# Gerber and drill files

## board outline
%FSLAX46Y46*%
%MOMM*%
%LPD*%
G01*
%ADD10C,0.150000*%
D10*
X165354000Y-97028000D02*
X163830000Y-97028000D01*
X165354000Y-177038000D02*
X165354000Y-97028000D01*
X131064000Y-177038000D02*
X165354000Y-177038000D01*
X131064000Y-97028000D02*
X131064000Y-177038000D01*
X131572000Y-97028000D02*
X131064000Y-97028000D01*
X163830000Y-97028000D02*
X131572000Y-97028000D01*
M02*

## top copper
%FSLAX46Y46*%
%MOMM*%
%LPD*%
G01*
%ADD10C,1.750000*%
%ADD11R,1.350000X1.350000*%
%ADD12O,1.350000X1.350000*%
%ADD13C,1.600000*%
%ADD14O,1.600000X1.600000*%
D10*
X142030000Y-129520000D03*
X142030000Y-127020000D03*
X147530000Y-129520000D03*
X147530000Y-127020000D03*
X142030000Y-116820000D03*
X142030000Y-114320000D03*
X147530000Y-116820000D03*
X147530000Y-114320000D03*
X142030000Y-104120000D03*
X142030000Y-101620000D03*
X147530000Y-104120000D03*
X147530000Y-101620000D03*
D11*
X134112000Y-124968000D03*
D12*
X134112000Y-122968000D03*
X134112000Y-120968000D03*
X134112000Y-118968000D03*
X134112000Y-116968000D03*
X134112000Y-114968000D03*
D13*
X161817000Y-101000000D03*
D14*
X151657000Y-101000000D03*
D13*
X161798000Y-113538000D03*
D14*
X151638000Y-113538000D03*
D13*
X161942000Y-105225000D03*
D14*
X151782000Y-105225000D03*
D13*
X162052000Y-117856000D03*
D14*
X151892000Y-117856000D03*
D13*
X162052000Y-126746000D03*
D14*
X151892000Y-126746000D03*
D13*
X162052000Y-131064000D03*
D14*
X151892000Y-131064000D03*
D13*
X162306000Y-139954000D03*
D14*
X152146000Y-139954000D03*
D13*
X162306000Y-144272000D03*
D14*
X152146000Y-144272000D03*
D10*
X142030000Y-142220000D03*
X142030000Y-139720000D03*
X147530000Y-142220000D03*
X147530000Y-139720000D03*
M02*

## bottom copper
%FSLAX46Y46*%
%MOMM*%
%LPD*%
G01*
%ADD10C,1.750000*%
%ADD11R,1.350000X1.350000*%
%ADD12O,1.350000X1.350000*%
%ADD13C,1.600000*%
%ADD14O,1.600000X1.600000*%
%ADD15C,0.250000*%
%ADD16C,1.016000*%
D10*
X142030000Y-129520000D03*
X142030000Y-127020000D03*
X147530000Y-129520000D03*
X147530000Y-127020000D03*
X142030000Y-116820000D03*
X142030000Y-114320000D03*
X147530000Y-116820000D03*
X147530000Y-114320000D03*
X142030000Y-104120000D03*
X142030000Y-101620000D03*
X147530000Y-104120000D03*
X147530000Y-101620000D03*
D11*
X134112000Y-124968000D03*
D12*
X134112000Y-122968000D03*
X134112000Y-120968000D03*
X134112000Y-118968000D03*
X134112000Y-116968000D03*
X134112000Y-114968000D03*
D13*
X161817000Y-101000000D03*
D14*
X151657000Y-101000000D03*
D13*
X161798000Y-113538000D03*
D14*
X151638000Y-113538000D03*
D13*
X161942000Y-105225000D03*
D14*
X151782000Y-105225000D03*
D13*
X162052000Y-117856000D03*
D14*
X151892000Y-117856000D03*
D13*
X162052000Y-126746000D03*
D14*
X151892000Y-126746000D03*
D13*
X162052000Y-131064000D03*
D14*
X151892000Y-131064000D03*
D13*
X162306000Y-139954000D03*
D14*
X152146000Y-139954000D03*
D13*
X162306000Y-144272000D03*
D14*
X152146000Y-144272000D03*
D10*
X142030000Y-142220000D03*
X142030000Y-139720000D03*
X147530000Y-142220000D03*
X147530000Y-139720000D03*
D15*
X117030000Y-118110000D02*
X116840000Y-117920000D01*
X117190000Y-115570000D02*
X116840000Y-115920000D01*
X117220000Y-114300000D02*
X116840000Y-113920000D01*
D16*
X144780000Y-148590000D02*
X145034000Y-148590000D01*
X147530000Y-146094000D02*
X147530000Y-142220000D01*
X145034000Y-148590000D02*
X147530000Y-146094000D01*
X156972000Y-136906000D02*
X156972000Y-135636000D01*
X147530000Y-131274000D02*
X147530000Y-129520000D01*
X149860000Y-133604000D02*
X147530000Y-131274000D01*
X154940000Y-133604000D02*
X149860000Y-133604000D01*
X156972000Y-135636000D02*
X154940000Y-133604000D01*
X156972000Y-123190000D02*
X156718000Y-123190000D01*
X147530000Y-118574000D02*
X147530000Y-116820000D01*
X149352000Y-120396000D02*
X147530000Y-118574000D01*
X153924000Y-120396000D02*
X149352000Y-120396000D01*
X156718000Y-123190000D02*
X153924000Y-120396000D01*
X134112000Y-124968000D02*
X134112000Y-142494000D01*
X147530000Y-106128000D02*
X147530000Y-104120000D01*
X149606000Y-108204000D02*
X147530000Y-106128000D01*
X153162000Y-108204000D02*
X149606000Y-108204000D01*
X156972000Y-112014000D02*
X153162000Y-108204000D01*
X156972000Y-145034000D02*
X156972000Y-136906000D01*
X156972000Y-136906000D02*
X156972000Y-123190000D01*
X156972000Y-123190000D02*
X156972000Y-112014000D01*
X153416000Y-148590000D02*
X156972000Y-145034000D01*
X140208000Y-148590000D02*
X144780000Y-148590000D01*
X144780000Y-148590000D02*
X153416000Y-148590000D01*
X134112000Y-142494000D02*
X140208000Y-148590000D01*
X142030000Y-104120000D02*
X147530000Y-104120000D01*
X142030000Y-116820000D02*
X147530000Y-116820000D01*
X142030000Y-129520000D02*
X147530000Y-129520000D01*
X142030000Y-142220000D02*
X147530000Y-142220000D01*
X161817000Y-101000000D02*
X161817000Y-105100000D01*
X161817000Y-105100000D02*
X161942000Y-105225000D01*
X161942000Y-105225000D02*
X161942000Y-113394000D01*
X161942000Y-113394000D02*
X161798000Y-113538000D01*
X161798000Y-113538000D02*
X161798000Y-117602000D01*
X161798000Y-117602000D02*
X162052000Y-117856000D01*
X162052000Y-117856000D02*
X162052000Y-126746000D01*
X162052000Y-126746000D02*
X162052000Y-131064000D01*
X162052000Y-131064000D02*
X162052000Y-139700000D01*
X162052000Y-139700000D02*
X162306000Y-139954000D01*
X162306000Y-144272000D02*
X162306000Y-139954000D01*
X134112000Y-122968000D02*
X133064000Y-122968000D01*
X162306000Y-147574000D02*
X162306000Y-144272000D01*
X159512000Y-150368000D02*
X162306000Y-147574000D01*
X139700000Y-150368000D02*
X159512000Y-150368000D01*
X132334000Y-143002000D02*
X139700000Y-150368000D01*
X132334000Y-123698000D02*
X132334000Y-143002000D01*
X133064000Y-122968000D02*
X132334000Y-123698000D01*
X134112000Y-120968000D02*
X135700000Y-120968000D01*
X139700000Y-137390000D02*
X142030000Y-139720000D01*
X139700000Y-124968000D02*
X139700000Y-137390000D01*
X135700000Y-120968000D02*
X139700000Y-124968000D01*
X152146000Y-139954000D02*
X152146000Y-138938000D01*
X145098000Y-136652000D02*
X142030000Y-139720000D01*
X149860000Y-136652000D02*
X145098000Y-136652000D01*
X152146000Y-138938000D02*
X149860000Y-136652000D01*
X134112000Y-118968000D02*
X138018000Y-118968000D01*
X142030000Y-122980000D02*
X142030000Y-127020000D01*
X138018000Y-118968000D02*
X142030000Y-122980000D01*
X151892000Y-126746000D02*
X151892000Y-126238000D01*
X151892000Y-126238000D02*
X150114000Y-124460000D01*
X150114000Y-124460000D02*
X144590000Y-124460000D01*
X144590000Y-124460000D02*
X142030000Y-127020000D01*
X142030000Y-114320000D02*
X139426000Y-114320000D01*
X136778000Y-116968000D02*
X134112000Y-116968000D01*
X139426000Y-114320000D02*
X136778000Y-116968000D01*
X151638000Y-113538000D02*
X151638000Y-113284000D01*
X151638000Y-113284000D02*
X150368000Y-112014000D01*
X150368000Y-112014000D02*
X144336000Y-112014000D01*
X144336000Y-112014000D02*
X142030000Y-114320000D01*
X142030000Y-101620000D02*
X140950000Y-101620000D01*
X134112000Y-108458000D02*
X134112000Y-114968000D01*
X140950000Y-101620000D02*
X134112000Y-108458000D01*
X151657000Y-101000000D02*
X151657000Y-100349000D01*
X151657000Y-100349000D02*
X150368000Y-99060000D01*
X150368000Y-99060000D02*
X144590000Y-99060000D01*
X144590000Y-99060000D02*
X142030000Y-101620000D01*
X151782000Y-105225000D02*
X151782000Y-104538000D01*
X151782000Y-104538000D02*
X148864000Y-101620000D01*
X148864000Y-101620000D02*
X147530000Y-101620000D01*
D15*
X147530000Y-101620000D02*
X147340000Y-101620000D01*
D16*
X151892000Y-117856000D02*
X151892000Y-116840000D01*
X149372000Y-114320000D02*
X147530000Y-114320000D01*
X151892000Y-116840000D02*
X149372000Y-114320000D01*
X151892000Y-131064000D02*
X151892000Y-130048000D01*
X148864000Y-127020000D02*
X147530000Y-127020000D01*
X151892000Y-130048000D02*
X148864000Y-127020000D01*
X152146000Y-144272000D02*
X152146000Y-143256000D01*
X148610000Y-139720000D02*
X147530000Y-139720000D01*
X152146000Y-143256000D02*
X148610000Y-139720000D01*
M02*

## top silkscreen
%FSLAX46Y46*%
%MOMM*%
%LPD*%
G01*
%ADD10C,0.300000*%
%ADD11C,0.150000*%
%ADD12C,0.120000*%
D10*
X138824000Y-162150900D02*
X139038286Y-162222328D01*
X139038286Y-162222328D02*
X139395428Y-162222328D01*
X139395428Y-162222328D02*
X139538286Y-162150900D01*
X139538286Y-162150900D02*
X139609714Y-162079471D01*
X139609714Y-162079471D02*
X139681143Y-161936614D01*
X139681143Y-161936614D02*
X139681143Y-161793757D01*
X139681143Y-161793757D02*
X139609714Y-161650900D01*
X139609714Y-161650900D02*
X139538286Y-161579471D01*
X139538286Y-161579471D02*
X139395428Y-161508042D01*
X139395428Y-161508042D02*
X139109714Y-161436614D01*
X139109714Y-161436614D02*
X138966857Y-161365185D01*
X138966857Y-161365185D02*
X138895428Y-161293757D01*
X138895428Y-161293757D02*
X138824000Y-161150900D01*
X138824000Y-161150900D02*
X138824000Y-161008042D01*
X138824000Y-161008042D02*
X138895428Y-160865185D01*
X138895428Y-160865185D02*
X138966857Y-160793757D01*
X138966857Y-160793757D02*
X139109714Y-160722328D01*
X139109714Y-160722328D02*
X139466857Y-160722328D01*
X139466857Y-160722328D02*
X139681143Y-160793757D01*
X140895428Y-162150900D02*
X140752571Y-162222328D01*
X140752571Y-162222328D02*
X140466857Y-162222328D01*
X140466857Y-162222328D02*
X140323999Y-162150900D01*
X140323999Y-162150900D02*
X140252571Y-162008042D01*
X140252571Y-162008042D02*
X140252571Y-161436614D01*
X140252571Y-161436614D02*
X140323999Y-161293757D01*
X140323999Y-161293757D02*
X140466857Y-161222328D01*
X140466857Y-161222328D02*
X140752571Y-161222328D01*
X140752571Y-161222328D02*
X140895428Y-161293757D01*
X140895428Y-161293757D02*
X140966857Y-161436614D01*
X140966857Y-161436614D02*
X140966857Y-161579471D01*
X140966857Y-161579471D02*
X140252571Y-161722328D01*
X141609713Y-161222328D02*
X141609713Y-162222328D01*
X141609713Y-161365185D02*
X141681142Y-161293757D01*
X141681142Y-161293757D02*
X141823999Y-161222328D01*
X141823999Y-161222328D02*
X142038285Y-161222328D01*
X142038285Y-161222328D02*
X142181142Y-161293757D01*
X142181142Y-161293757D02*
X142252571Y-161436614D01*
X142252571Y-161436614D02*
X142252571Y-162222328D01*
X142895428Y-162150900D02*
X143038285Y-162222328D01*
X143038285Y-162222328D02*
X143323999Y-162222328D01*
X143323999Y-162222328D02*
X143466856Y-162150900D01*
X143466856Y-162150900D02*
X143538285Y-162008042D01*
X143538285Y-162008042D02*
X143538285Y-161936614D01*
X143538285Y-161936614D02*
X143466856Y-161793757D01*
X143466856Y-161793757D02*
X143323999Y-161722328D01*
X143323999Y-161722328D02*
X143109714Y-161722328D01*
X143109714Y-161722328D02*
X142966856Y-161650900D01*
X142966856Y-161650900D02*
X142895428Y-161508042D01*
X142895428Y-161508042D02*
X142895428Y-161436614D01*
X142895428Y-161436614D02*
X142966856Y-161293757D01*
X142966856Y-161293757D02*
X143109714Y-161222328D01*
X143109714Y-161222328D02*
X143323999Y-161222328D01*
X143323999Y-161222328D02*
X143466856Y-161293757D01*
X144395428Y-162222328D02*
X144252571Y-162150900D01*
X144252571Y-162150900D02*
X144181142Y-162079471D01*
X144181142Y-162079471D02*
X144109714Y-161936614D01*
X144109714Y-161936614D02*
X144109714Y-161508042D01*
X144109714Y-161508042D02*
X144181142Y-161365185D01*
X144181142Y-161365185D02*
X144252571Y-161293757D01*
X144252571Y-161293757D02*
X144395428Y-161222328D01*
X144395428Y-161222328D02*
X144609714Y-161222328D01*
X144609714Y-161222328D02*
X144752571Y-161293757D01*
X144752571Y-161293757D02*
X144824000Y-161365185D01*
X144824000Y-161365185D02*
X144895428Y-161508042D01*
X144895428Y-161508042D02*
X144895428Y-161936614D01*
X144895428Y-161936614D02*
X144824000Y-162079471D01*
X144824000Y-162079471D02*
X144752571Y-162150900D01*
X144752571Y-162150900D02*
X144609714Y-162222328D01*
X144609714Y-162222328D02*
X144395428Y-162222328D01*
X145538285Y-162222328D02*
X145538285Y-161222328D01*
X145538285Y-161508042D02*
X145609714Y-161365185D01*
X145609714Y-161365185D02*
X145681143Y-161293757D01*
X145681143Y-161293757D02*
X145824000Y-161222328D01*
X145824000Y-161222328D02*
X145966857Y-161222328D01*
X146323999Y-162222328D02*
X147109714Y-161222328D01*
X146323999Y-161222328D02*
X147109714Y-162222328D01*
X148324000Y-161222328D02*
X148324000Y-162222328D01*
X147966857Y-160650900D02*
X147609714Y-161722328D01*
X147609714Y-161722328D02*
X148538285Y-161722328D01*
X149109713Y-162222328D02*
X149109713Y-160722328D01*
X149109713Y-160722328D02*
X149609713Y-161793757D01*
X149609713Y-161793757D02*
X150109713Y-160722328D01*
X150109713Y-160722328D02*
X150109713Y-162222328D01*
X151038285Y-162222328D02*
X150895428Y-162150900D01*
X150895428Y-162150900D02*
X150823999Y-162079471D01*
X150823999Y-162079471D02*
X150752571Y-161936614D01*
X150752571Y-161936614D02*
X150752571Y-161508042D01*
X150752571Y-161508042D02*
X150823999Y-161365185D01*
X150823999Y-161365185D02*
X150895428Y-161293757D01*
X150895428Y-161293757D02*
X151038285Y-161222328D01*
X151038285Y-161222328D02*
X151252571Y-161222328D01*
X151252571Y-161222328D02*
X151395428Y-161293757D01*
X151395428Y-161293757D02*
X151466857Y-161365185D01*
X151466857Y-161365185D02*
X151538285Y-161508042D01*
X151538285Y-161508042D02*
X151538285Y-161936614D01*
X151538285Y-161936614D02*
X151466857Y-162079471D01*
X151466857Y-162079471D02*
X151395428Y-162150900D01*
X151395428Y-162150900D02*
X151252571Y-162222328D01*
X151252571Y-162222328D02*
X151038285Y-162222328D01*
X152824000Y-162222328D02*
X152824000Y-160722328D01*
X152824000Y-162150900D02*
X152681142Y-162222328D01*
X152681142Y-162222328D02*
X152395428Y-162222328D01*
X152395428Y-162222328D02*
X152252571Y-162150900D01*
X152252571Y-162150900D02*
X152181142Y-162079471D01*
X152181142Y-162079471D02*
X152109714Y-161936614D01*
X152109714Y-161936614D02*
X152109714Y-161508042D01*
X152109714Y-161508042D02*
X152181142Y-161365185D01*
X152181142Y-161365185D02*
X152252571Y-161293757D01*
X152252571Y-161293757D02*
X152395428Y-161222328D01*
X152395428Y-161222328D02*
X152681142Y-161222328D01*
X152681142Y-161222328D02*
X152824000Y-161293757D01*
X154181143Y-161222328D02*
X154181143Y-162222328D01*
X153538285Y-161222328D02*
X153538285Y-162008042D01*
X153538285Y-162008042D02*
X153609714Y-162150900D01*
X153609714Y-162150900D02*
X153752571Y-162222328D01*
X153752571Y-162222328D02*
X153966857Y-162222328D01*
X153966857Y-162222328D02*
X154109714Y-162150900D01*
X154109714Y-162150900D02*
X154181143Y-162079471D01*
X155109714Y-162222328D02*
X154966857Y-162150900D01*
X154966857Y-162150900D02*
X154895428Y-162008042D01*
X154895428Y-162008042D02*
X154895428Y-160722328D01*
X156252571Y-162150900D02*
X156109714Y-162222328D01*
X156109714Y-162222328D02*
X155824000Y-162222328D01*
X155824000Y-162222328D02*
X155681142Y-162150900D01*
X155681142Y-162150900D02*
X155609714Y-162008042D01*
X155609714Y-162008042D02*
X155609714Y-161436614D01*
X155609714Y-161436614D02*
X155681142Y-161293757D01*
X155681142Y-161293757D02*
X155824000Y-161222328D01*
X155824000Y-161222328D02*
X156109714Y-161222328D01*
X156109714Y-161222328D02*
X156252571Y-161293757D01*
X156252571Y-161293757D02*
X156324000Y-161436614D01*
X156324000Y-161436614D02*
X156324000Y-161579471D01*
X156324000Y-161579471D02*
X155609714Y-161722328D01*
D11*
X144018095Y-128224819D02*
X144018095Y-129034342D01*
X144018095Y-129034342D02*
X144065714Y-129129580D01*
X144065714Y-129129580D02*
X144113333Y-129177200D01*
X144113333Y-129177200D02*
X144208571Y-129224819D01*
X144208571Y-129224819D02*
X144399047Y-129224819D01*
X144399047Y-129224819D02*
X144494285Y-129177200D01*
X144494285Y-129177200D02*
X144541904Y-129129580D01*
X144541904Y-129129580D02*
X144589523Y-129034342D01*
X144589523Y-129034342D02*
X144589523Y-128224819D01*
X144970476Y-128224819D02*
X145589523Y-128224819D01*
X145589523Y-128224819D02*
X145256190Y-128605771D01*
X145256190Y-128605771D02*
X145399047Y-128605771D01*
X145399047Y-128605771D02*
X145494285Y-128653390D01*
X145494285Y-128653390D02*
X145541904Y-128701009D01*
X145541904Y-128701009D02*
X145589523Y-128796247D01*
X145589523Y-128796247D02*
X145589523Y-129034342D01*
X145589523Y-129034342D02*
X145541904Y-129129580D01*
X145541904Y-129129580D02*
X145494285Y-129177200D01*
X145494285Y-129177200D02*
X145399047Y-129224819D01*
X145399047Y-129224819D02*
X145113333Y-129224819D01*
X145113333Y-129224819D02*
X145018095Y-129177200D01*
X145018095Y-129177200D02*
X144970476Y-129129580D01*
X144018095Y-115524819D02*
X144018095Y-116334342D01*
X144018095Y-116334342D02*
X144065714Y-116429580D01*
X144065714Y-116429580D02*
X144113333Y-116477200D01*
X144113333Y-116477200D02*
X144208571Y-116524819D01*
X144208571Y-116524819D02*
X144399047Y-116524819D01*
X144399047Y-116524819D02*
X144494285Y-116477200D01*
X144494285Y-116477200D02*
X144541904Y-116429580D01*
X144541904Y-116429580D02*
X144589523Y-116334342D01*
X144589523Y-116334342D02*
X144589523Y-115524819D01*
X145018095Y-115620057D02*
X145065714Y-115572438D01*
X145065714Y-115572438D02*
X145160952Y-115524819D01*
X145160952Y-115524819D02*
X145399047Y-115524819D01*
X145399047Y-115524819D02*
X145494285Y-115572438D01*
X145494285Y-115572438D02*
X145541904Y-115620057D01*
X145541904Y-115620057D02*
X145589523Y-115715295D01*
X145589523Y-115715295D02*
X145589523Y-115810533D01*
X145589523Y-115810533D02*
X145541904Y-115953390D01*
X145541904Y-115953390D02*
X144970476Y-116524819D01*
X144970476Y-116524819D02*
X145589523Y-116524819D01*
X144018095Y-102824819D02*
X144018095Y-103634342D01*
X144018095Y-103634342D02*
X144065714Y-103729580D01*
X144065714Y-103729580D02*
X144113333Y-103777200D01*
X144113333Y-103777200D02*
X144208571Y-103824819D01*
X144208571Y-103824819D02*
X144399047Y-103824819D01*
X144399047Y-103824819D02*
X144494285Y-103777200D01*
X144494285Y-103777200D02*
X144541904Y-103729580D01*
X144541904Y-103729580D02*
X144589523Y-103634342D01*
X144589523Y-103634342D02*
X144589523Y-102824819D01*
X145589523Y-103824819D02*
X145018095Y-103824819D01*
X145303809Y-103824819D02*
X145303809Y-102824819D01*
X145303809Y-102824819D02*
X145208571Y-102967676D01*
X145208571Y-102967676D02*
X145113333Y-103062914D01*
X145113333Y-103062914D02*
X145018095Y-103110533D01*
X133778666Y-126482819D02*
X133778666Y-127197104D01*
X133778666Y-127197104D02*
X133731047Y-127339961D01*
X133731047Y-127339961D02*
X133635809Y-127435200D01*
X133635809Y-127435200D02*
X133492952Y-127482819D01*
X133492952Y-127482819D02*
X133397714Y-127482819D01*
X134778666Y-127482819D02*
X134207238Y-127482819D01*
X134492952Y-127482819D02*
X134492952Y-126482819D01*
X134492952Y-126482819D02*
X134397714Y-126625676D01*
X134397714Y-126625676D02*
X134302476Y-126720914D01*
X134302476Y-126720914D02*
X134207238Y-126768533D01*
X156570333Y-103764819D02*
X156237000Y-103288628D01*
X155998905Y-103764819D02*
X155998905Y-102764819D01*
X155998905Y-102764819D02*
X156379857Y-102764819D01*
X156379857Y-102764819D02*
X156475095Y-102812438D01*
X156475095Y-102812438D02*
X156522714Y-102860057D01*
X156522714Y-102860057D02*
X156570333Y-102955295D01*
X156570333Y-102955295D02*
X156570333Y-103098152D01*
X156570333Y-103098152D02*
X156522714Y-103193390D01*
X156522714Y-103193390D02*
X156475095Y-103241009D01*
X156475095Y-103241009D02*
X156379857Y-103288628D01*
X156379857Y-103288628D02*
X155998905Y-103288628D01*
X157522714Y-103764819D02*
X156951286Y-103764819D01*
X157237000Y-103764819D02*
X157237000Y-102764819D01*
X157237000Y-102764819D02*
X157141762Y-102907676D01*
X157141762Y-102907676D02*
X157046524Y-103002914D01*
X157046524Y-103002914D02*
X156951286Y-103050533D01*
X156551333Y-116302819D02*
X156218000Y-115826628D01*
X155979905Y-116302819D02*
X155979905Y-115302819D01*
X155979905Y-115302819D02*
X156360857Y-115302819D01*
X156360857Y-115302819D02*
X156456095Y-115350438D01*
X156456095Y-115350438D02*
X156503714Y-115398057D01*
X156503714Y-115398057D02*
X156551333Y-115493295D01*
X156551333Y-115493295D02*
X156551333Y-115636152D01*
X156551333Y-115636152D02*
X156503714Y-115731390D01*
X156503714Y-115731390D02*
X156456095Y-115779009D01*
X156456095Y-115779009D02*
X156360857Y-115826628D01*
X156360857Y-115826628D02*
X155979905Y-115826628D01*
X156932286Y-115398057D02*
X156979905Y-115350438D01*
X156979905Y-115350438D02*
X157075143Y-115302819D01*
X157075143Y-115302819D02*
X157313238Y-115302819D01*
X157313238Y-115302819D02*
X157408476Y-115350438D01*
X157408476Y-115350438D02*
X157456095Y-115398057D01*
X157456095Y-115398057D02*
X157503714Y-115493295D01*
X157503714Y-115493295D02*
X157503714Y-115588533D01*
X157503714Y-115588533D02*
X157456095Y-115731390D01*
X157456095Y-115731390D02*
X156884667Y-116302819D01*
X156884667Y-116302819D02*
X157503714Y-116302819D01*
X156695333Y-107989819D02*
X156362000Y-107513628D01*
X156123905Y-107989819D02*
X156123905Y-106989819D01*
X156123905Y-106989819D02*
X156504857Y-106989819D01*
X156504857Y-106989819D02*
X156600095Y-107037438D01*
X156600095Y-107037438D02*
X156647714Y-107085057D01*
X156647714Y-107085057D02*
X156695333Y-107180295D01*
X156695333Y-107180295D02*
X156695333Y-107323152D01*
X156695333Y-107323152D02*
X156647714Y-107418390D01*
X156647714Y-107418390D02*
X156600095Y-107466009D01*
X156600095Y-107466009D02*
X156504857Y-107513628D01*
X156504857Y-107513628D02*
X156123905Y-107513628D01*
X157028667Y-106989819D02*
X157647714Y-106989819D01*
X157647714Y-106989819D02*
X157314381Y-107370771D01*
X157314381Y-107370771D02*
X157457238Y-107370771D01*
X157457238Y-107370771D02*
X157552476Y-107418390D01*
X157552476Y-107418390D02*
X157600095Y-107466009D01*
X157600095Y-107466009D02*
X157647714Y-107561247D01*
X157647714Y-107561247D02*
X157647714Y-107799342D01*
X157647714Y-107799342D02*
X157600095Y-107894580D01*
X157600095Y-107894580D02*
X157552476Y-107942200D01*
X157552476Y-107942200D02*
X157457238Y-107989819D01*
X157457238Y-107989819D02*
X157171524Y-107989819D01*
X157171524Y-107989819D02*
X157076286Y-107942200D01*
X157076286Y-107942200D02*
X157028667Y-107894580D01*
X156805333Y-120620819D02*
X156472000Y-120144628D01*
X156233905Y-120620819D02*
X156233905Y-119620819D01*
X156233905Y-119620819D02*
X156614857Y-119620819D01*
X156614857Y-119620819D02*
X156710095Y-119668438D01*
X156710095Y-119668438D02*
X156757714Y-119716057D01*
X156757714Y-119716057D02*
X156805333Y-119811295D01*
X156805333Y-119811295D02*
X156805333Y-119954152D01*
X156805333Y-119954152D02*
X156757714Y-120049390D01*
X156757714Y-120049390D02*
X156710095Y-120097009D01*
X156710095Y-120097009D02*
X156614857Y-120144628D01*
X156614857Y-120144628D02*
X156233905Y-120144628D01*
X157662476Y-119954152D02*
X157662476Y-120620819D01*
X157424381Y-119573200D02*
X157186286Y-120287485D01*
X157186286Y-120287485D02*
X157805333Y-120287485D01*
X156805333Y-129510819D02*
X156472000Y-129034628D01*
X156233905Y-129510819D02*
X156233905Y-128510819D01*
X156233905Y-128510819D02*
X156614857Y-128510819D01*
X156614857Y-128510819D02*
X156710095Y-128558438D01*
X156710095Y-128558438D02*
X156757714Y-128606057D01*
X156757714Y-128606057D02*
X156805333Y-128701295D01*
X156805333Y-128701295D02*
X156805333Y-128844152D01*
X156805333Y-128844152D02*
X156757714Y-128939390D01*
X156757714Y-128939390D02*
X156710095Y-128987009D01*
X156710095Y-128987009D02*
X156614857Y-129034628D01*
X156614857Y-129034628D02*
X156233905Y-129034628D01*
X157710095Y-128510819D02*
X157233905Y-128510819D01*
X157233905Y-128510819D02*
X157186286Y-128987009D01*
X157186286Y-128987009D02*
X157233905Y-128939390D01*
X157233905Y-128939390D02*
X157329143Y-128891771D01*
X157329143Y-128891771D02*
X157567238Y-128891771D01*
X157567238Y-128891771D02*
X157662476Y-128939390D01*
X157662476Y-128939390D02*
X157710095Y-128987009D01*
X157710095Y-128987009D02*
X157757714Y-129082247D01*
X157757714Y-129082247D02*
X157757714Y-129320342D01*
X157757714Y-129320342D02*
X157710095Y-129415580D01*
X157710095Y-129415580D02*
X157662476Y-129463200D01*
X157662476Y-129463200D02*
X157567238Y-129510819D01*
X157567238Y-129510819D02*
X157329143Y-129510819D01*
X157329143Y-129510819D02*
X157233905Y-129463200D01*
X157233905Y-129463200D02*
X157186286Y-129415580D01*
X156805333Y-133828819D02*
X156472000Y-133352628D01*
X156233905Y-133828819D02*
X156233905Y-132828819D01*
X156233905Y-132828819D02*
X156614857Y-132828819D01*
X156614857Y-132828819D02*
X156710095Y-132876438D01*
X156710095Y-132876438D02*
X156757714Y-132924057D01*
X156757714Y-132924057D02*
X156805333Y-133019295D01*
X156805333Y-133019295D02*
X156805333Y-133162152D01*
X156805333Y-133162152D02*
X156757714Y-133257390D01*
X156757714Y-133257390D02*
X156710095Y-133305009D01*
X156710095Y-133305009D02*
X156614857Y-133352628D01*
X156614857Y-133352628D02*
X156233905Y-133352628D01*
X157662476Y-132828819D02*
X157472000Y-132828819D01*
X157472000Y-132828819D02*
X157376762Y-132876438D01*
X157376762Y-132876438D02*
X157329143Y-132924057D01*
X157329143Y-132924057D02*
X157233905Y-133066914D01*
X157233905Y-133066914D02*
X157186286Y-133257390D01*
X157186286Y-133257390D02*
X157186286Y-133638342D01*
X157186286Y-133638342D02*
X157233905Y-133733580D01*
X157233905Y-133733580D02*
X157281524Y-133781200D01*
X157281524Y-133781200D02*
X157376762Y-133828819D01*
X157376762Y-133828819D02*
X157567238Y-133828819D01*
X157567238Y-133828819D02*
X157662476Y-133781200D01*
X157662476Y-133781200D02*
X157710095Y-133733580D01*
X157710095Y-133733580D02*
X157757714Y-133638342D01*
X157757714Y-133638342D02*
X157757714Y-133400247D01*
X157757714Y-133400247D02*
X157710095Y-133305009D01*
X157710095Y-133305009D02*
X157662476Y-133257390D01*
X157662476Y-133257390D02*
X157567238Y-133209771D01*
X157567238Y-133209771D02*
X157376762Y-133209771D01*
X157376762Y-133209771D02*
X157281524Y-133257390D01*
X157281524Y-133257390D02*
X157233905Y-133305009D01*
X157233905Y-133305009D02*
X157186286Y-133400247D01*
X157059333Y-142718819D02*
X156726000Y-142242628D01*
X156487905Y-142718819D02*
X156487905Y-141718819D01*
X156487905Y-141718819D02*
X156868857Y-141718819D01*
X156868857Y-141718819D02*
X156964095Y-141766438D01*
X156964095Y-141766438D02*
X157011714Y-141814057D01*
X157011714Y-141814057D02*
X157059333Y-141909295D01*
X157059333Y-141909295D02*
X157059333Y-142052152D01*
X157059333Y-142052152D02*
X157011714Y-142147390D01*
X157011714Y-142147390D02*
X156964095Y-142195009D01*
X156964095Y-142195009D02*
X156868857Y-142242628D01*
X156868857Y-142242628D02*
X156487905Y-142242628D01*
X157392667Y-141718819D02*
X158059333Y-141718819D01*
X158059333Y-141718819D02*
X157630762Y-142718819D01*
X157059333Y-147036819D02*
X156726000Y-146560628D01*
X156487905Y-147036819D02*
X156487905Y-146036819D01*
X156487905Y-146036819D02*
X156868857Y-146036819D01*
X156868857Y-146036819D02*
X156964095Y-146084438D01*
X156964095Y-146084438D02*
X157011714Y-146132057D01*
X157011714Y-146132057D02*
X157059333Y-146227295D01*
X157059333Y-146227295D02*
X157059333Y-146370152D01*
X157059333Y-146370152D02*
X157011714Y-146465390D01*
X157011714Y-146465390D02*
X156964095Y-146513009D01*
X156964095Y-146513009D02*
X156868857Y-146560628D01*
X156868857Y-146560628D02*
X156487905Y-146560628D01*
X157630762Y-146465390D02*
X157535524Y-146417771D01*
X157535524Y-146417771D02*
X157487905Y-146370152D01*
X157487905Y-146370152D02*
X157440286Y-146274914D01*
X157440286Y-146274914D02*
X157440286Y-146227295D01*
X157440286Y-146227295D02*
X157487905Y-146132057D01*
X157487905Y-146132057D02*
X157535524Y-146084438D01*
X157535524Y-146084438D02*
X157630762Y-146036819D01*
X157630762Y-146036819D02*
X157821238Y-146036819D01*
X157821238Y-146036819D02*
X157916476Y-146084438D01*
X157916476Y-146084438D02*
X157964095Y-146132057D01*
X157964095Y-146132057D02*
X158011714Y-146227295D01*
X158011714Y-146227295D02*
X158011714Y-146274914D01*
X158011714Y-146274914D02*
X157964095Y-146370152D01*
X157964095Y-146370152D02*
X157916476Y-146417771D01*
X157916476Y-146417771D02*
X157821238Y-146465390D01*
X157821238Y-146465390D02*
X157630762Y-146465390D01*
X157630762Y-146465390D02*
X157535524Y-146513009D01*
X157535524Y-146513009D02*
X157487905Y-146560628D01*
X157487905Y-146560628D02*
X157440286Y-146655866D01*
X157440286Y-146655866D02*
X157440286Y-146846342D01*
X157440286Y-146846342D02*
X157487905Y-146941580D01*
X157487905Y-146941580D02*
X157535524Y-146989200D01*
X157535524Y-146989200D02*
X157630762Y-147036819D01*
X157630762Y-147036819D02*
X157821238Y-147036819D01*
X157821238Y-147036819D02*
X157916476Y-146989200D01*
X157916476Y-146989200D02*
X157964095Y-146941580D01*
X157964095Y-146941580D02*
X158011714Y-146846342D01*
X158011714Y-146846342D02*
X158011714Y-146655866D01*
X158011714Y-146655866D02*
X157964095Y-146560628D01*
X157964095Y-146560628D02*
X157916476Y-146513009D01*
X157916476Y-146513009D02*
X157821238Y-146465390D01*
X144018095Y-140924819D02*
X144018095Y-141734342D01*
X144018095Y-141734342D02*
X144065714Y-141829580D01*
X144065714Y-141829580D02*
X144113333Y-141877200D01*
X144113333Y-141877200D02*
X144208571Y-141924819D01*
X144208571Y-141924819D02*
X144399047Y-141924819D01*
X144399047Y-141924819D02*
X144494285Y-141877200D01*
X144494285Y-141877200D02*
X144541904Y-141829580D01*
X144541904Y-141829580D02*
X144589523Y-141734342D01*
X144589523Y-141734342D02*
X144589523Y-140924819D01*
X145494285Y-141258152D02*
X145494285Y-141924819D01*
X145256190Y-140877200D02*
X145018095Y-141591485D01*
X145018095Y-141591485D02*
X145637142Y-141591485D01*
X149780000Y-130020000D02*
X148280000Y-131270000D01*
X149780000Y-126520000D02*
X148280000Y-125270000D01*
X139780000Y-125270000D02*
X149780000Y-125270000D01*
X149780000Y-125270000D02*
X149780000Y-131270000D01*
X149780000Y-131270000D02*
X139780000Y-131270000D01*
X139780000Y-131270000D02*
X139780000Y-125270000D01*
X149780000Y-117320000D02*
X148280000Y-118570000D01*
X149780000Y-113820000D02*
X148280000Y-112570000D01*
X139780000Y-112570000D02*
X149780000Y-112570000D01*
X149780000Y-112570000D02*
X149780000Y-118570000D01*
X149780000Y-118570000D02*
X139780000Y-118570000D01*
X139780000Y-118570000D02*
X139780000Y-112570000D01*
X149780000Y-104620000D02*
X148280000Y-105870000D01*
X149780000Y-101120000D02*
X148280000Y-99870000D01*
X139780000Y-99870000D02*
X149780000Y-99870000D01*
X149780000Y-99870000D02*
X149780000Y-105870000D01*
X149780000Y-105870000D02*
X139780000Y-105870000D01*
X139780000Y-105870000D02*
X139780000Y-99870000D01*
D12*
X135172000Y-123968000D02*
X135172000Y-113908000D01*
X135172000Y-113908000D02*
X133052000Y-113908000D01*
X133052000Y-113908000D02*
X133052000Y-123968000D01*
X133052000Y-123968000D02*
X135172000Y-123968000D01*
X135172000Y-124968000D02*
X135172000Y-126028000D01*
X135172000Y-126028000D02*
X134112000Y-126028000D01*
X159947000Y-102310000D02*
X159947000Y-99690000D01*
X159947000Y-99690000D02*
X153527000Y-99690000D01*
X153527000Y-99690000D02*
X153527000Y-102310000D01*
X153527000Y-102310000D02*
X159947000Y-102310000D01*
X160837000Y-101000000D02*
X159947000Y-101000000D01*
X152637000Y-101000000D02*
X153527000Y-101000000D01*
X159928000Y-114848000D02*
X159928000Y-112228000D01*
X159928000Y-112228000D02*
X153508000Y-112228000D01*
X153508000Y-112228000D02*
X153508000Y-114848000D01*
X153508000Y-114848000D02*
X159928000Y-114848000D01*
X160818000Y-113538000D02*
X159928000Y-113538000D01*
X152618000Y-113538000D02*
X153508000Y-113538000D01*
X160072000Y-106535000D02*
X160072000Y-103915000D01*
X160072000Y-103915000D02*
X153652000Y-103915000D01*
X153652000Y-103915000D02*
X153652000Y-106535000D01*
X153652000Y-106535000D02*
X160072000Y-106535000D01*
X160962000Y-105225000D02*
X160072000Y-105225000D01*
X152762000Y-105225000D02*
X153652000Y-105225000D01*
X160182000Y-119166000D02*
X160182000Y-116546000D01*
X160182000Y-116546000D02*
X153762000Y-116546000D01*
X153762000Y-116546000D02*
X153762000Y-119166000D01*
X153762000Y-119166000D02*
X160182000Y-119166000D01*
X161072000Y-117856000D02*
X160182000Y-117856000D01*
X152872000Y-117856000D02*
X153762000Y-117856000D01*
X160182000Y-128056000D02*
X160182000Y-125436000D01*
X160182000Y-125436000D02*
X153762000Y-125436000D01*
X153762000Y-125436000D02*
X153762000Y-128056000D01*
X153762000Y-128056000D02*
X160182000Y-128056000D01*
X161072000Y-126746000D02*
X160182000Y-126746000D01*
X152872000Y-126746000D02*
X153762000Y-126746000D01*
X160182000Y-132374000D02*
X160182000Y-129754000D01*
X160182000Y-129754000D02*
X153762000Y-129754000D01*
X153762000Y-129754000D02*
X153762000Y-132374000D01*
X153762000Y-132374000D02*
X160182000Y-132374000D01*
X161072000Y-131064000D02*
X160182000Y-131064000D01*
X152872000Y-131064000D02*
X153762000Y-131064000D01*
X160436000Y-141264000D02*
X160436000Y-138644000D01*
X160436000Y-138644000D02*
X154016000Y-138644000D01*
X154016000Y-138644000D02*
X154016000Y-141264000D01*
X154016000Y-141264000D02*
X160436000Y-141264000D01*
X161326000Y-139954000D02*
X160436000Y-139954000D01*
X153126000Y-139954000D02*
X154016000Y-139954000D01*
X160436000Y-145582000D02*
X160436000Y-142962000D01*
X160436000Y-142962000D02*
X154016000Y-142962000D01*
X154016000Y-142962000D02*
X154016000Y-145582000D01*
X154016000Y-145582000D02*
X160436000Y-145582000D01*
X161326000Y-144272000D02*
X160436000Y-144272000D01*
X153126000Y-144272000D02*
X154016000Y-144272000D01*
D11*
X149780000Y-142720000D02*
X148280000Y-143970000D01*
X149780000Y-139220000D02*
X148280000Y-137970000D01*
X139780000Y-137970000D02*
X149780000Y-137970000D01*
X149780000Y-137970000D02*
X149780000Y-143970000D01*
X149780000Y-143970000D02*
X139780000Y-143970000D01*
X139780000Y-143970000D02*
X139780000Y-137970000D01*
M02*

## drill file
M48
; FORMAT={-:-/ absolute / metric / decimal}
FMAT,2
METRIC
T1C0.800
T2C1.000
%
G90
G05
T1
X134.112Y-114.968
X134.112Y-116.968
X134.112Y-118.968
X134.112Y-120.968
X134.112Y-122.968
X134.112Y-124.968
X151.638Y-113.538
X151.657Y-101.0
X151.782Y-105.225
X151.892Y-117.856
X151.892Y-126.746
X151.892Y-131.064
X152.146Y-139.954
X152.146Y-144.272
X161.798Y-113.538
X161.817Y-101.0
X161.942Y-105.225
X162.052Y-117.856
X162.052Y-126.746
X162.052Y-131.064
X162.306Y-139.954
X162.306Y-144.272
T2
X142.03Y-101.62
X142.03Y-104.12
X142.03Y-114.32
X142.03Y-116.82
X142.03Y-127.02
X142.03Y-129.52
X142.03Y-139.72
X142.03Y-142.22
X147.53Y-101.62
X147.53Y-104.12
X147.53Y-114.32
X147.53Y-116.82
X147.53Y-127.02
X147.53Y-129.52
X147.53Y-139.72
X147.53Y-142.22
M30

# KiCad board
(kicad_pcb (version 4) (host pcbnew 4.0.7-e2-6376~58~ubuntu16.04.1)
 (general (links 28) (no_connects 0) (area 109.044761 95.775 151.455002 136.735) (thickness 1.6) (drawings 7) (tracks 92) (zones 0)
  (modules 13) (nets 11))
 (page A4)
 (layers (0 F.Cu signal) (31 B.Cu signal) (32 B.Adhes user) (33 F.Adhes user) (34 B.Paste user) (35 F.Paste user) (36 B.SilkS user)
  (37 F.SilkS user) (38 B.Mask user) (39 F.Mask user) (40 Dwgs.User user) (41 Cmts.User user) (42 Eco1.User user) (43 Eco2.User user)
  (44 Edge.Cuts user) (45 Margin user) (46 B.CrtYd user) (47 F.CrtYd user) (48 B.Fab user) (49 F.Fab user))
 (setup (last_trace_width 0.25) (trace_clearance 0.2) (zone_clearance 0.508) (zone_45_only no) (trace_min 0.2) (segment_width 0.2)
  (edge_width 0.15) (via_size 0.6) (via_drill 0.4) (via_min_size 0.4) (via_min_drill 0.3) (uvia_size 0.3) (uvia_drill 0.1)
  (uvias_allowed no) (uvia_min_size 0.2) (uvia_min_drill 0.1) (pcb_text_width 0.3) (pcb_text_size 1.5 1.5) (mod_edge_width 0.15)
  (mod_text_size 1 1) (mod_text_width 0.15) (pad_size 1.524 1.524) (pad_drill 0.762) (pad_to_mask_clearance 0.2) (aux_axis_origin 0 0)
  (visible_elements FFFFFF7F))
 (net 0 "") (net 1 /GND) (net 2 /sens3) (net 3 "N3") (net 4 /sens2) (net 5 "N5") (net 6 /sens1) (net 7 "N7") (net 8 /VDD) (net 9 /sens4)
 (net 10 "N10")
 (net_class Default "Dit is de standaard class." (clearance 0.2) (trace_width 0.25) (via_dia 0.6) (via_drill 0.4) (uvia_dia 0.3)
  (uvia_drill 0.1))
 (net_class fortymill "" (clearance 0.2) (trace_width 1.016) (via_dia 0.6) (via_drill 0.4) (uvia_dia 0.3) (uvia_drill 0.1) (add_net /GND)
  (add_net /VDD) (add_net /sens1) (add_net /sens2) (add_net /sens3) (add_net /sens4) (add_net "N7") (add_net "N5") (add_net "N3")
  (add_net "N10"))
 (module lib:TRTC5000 (layer F.Cu) (at 144.78 128.27)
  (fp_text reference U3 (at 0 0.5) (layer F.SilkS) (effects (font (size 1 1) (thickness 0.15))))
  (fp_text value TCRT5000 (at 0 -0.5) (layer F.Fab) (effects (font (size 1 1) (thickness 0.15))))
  (fp_line (start 5 1.75) (end 3.5 3) (layer F.SilkS) (width 0.15))
  (fp_line (start 5 -1.75) (end 3.5 -3) (layer F.SilkS) (width 0.15))
  (fp_line (start -5 -3) (end 5 -3) (layer F.SilkS) (width 0.15))
  (fp_line (start 5 -3) (end 5 3) (layer F.SilkS) (width 0.15))
  (fp_line (start 5 3) (end -5 3) (layer F.SilkS) (width 0.15))
  (fp_line (start -5 3) (end -5 -3) (layer F.SilkS) (width 0.15))
  (pad 2 thru_hole circle (at -2.75 1.25) (size 1.75 1.75) (drill 1) (layers *.Cu *.Mask) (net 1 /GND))
  (pad 1 thru_hole circle (at -2.75 -1.25) (size 1.75 1.75) (drill 1) (layers *.Cu *.Mask) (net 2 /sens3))
  (pad 4 thru_hole circle (at 2.75 1.25) (size 1.75 1.75) (drill 1) (layers *.Cu *.Mask) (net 1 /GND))
  (pad 3 thru_hole circle (at 2.75 -1.25) (size 1.75 1.75) (drill 1) (layers *.Cu *.Mask) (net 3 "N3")))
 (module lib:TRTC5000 (layer F.Cu) (at 144.78 115.57)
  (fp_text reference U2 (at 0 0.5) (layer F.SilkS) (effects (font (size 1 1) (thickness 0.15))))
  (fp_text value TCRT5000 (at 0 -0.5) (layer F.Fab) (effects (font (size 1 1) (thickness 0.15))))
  (fp_line (start 5 1.75) (end 3.5 3) (layer F.SilkS) (width 0.15))
  (fp_line (start 5 -1.75) (end 3.5 -3) (layer F.SilkS) (width 0.15))
  (fp_line (start -5 -3) (end 5 -3) (layer F.SilkS) (width 0.15))
  (fp_line (start 5 -3) (end 5 3) (layer F.SilkS) (width 0.15))
  (fp_line (start 5 3) (end -5 3) (layer F.SilkS) (width 0.15))
  (fp_line (start -5 3) (end -5 -3) (layer F.SilkS) (width 0.15))
  (pad 2 thru_hole circle (at -2.75 1.25) (size 1.75 1.75) (drill 1) (layers *.Cu *.Mask) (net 1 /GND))
  (pad 1 thru_hole circle (at -2.75 -1.25) (size 1.75 1.75) (drill 1) (layers *.Cu *.Mask) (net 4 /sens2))
  (pad 4 thru_hole circle (at 2.75 1.25) (size 1.75 1.75) (drill 1) (layers *.Cu *.Mask) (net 1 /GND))
  (pad 3 thru_hole circle (at 2.75 -1.25) (size 1.75 1.75) (drill 1) (layers *.Cu *.Mask) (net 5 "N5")))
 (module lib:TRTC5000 (layer F.Cu) (at 144.78 102.87)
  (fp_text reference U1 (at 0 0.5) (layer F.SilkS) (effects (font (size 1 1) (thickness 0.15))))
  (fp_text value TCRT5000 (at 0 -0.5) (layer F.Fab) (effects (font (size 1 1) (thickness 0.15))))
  (fp_line (start 5 1.75) (end 3.5 3) (layer F.SilkS) (width 0.15))
  (fp_line (start 5 -1.75) (end 3.5 -3) (layer F.SilkS) (width 0.15))
  (fp_line (start -5 -3) (end 5 -3) (layer F.SilkS) (width 0.15))
  (fp_line (start 5 -3) (end 5 3) (layer F.SilkS) (width 0.15))
  (fp_line (start 5 3) (end -5 3) (layer F.SilkS) (width 0.15))
  (fp_line (start -5 3) (end -5 -3) (layer F.SilkS) (width 0.15))
  (pad 2 thru_hole circle (at -2.75 1.25) (size 1.75 1.75) (drill 1) (layers *.Cu *.Mask) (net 1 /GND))
  (pad 1 thru_hole circle (at -2.75 -1.25) (size 1.75 1.75) (drill 1) (layers *.Cu *.Mask) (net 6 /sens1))
  (pad 4 thru_hole circle (at 2.75 1.25) (size 1.75 1.75) (drill 1) (layers *.Cu *.Mask) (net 1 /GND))
  (pad 3 thru_hole circle (at 2.75 -1.25) (size 1.75 1.75) (drill 1) (layers *.Cu *.Mask) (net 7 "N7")))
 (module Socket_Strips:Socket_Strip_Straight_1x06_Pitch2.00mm (layer F.Cu) (at 134.112 124.968 180)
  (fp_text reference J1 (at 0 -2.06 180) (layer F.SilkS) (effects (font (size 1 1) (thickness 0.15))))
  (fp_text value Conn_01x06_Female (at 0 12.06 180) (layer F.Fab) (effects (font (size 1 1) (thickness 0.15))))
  (fp_line (start -1.06 1) (end -1.06 11.06) (layer F.SilkS) (width 0.12))
  (fp_line (start -1.06 11.06) (end 1.06 11.06) (layer F.SilkS) (width 0.12))
  (fp_line (start 1.06 11.06) (end 1.06 1) (layer F.SilkS) (width 0.12))
  (fp_line (start 1.06 1) (end -1.06 1) (layer F.SilkS) (width 0.12))
  (fp_line (start -1.06 0) (end -1.06 -1.06) (layer F.SilkS) (width 0.12))
  (fp_line (start -1.06 -1.06) (end 0 -1.06) (layer F.SilkS) (width 0.12))
  (pad 1 thru_hole rect (at 0 0 180) (size 1.35 1.35) (drill 0.8) (layers *.Cu *.Mask) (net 1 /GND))
  (pad 2 thru_hole oval (at 0 2 180) (size 1.35 1.35) (drill 0.8) (layers *.Cu *.Mask) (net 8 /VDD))
  (pad 3 thru_hole oval (at 0 4 180) (size 1.35 1.35) (drill 0.8) (layers *.Cu *.Mask) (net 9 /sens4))
  (pad 4 thru_hole oval (at 0 6 180) (size 1.35 1.35) (drill 0.8) (layers *.Cu *.Mask) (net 2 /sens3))
  (pad 5 thru_hole oval (at 0 8 180) (size 1.35 1.35) (drill 0.8) (layers *.Cu *.Mask) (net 4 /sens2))
  (pad 6 thru_hole oval (at 0 10 180) (size 1.35 1.35) (drill 0.8) (layers *.Cu *.Mask) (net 6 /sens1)))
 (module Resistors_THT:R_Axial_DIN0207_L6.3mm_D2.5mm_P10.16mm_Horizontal (layer F.Cu) (at 161.817 101 180)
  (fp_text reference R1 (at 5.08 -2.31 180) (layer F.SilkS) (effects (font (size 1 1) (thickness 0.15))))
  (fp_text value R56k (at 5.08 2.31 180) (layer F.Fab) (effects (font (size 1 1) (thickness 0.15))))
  (fp_line (start 1.87 -1.31) (end 1.87 1.31) (layer F.SilkS) (width 0.12))
  (fp_line (start 1.87 1.31) (end 8.29 1.31) (layer F.SilkS) (width 0.12))
  (fp_line (start 8.29 1.31) (end 8.29 -1.31) (layer F.SilkS) (width 0.12))
  (fp_line (start 8.29 -1.31) (end 1.87 -1.31) (layer F.SilkS) (width 0.12))
  (fp_line (start 0.98 0) (end 1.87 0) (layer F.SilkS) (width 0.12))
  (fp_line (start 9.18 0) (end 8.29 0) (layer F.SilkS) (width 0.12))
  (pad 1 thru_hole circle (at 0 0 180) (size 1.6 1.6) (drill 0.8) (layers *.Cu *.Mask) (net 8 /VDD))
  (pad 2 thru_hole oval (at 10.16 0 180) (size 1.6 1.6) (drill 0.8) (layers *.Cu *.Mask) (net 6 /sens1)))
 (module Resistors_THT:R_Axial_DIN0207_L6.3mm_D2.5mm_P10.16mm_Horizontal (layer F.Cu) (at 161.798 113.538 180)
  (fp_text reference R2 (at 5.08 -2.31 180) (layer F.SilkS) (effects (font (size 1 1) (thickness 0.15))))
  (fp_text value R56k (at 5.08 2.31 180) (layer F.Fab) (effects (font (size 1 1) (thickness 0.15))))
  (fp_line (start 1.87 -1.31) (end 1.87 1.31) (layer F.SilkS) (width 0.12))
  (fp_line (start 1.87 1.31) (end 8.29 1.31) (layer F.SilkS) (width 0.12))
  (fp_line (start 8.29 1.31) (end 8.29 -1.31) (layer F.SilkS) (width 0.12))
  (fp_line (start 8.29 -1.31) (end 1.87 -1.31) (layer F.SilkS) (width 0.12))
  (fp_line (start 0.98 0) (end 1.87 0) (layer F.SilkS) (width 0.12))
  (fp_line (start 9.18 0) (end 8.29 0) (layer F.SilkS) (width 0.12))
  (pad 1 thru_hole circle (at 0 0 180) (size 1.6 1.6) (drill 0.8) (layers *.Cu *.Mask) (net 8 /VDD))
  (pad 2 thru_hole oval (at 10.16 0 180) (size 1.6 1.6) (drill 0.8) (layers *.Cu *.Mask) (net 4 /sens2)))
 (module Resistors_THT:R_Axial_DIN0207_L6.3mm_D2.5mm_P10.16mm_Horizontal (layer F.Cu) (at 161.942 105.225 180)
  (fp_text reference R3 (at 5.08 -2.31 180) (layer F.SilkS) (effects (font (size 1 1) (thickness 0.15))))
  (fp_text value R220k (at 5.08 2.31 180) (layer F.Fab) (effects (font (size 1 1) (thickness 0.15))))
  (fp_line (start 1.87 -1.31) (end 1.87 1.31) (layer F.SilkS) (width 0.12))
  (fp_line (start 1.87 1.31) (end 8.29 1.31) (layer F.SilkS) (width 0.12))
  (fp_line (start 8.29 1.31) (end 8.29 -1.31) (layer F.SilkS) (width 0.12))
  (fp_line (start 8.29 -1.31) (end 1.87 -1.31) (layer F.SilkS) (width 0.12))
  (fp_line (start 0.98 0) (end 1.87 0) (layer F.SilkS) (width 0.12))
  (fp_line (start 9.18 0) (end 8.29 0) (layer F.SilkS) (width 0.12))
  (pad 1 thru_hole circle (at 0 0 180) (size 1.6 1.6) (drill 0.8) (layers *.Cu *.Mask) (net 8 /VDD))
  (pad 2 thru_hole oval (at 10.16 0 180) (size 1.6 1.6) (drill 0.8) (layers *.Cu *.Mask) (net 7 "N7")))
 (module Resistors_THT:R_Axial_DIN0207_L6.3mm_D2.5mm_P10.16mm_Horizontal (layer F.Cu) (at 162.052 117.856 180)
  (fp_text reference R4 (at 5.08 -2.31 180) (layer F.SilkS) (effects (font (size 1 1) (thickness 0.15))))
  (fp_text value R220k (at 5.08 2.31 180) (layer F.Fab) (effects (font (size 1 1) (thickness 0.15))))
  (fp_line (start 1.87 -1.31) (end 1.87 1.31) (layer F.SilkS) (width 0.12))
  (fp_line (start 1.87 1.31) (end 8.29 1.31) (layer F.SilkS) (width 0.12))
  (fp_line (start 8.29 1.31) (end 8.29 -1.31) (layer F.SilkS) (width 0.12))
  (fp_line (start 8.29 -1.31) (end 1.87 -1.31) (layer F.SilkS) (width 0.12))
  (fp_line (start 0.98 0) (end 1.87 0) (layer F.SilkS) (width 0.12))
  (fp_line (start 9.18 0) (end 8.29 0) (layer F.SilkS) (width 0.12))
  (pad 1 thru_hole circle (at 0 0 180) (size 1.6 1.6) (drill 0.8) (layers *.Cu *.Mask) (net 8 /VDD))
  (pad 2 thru_hole oval (at 10.16 0 180) (size 1.6 1.6) (drill 0.8) (layers *.Cu *.Mask) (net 5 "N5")))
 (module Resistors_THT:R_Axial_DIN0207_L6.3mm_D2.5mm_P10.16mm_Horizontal (layer F.Cu) (at 162.052 126.746 180)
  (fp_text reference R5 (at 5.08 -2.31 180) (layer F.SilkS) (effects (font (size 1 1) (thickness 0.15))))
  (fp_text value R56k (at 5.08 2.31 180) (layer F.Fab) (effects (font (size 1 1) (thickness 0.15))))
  (fp_line (start 1.87 -1.31) (end 1.87 1.31) (layer F.SilkS) (width 0.12))
  (fp_line (start 1.87 1.31) (end 8.29 1.31) (layer F.SilkS) (width 0.12))
  (fp_line (start 8.29 1.31) (end 8.29 -1.31) (layer F.SilkS) (width 0.12))
  (fp_line (start 8.29 -1.31) (end 1.87 -1.31) (layer F.SilkS) (width 0.12))
  (fp_line (start 0.98 0) (end 1.87 0) (layer F.SilkS) (width 0.12))
  (fp_line (start 9.18 0) (end 8.29 0) (layer F.SilkS) (width 0.12))
  (pad 1 thru_hole circle (at 0 0 180) (size 1.6 1.6) (drill 0.8) (layers *.Cu *.Mask) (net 8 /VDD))
  (pad 2 thru_hole oval (at 10.16 0 180) (size 1.6 1.6) (drill 0.8) (layers *.Cu *.Mask) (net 2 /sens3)))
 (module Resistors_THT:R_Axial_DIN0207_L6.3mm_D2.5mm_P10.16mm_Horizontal (layer F.Cu) (at 162.052 131.064 180)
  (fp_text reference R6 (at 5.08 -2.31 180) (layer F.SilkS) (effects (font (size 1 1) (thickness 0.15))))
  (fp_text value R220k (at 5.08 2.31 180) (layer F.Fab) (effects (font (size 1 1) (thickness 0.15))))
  (fp_line (start 1.87 -1.31) (end 1.87 1.31) (layer F.SilkS) (width 0.12))
  (fp_line (start 1.87 1.31) (end 8.29 1.31) (layer F.SilkS) (width 0.12))
  (fp_line (start 8.29 1.31) (end 8.29 -1.31) (layer F.SilkS) (width 0.12))
  (fp_line (start 8.29 -1.31) (end 1.87 -1.31) (layer F.SilkS) (width 0.12))
  (fp_line (start 0.98 0) (end 1.87 0) (layer F.SilkS) (width 0.12))
  (fp_line (start 9.18 0) (end 8.29 0) (layer F.SilkS) (width 0.12))
  (pad 1 thru_hole circle (at 0 0 180) (size 1.6 1.6) (drill 0.8) (layers *.Cu *.Mask) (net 8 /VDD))
  (pad 2 thru_hole oval (at 10.16 0 180) (size 1.6 1.6) (drill 0.8) (layers *.Cu *.Mask) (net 3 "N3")))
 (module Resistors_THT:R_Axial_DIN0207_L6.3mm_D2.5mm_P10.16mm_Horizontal (layer F.Cu) (at 162.306 139.954 180)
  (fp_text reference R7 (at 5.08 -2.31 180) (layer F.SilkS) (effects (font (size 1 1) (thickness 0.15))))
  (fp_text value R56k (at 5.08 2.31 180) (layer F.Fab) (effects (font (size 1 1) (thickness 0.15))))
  (fp_line (start 1.87 -1.31) (end 1.87 1.31) (layer F.SilkS) (width 0.12))
  (fp_line (start 1.87 1.31) (end 8.29 1.31) (layer F.SilkS) (width 0.12))
  (fp_line (start 8.29 1.31) (end 8.29 -1.31) (layer F.SilkS) (width 0.12))
  (fp_line (start 8.29 -1.31) (end 1.87 -1.31) (layer F.SilkS) (width 0.12))
  (fp_line (start 0.98 0) (end 1.87 0) (layer F.SilkS) (width 0.12))
  (fp_line (start 9.18 0) (end 8.29 0) (layer F.SilkS) (width 0.12))
  (pad 1 thru_hole circle (at 0 0 180) (size 1.6 1.6) (drill 0.8) (layers *.Cu *.Mask) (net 8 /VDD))
  (pad 2 thru_hole oval (at 10.16 0 180) (size 1.6 1.6) (drill 0.8) (layers *.Cu *.Mask) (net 9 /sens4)))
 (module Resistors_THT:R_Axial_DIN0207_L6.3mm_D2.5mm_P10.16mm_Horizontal (layer F.Cu) (at 162.306 144.272 180)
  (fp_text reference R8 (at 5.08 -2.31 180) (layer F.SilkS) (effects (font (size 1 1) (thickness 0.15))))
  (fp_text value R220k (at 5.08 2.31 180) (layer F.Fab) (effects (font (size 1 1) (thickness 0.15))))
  (fp_line (start 1.87 -1.31) (end 1.87 1.31) (layer F.SilkS) (width 0.12))
  (fp_line (start 1.87 1.31) (end 8.29 1.31) (layer F.SilkS) (width 0.12))
  (fp_line (start 8.29 1.31) (end 8.29 -1.31) (layer F.SilkS) (width 0.12))
  (fp_line (start 8.29 -1.31) (end 1.87 -1.31) (layer F.SilkS) (width 0.12))
  (fp_line (start 0.98 0) (end 1.87 0) (layer F.SilkS) (width 0.12))
  (fp_line (start 9.18 0) (end 8.29 0) (layer F.SilkS) (width 0.12))
  (pad 1 thru_hole circle (at 0 0 180) (size 1.6 1.6) (drill 0.8) (layers *.Cu *.Mask) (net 8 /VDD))
  (pad 2 thru_hole oval (at 10.16 0 180) (size 1.6 1.6) (drill 0.8) (layers *.Cu *.Mask) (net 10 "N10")))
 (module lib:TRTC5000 (layer F.Cu) (at 144.78 140.97)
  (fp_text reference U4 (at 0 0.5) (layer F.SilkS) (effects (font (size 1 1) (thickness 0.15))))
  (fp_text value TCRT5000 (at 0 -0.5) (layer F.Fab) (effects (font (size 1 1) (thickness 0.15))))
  (fp_line (start 5 1.75) (end 3.5 3) (layer F.SilkS) (width 0.15))
  (fp_line (start 5 -1.75) (end 3.5 -3) (layer F.SilkS) (width 0.15))
  (fp_line (start -5 -3) (end 5 -3) (layer F.SilkS) (width 0.15))
  (fp_line (start 5 -3) (end 5 3) (layer F.SilkS) (width 0.15))
  (fp_line (start 5 3) (end -5 3) (layer F.SilkS) (width 0.15))
  (fp_line (start -5 3) (end -5 -3) (layer F.SilkS) (width 0.15))
  (pad 2 thru_hole circle (at -2.75 1.25) (size 1.75 1.75) (drill 1) (layers *.Cu *.Mask) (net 1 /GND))
  (pad 1 thru_hole circle (at -2.75 -1.25) (size 1.75 1.75) (drill 1) (layers *.Cu *.Mask) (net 9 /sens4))
  (pad 4 thru_hole circle (at 2.75 1.25) (size 1.75 1.75) (drill 1) (layers *.Cu *.Mask) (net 1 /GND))
  (pad 3 thru_hole circle (at 2.75 -1.25) (size 1.75 1.75) (drill 1) (layers *.Cu *.Mask) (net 10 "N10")))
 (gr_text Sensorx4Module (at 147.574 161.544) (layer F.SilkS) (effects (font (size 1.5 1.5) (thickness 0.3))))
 (gr_line (start 165.354 97.028) (end 163.83 97.028) (angle 90) (layer Edge.Cuts) (width 0.15))
 (gr_line (start 165.354 177.038) (end 165.354 97.028) (angle 90) (layer Edge.Cuts) (width 0.15))
 (gr_line (start 131.064 177.038) (end 165.354 177.038) (angle 90) (layer Edge.Cuts) (width 0.15))
 (gr_line (start 131.064 97.028) (end 131.064 177.038) (angle 90) (layer Edge.Cuts) (width 0.15))
 (gr_line (start 131.572 97.028) (end 131.064 97.028) (angle 90) (layer Edge.Cuts) (width 0.15))
 (gr_line (start 163.83 97.028) (end 131.572 97.028) (angle 90) (layer Edge.Cuts) (width 0.15))
 (segment (start 117.03 118.11) (end 116.84 117.92) (width 0.25) (layer B.Cu) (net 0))
 (segment (start 117.19 115.57) (end 116.84 115.92) (width 0.25) (layer B.Cu) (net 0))
 (segment (start 117.22 114.3) (end 116.84 113.92) (width 0.25) (layer B.Cu) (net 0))
 (segment (start 144.78 148.59) (end 145.034 148.59) (width 1.016) (layer B.Cu) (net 1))
 (segment (start 147.53 146.094) (end 147.53 142.22) (width 1.016) (layer B.Cu) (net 1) (status 800000))
 (segment (start 145.034 148.59) (end 147.53 146.094) (width 1.016) (layer B.Cu) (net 1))
 (segment (start 156.972 136.906) (end 156.972 135.636) (width 1.016) (layer B.Cu) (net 1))
 (segment (start 147.53 131.274) (end 147.53 129.52) (width 1.016) (layer B.Cu) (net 1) (status 800000))
 (segment (start 149.86 133.604) (end 147.53 131.274) (width 1.016) (layer B.Cu) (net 1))
 (segment (start 154.94 133.604) (end 149.86 133.604) (width 1.016) (layer B.Cu) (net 1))
 (segment (start 156.972 135.636) (end 154.94 133.604) (width 1.016) (layer B.Cu) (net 1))
 (segment (start 156.972 123.19) (end 156.718 123.19) (width 1.016) (layer B.Cu) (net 1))
 (segment (start 147.53 118.574) (end 147.53 116.82) (width 1.016) (layer B.Cu) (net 1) (status 800000))
 (segment (start 149.352 120.396) (end 147.53 118.574) (width 1.016) (layer B.Cu) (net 1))
 (segment (start 153.924 120.396) (end 149.352 120.396) (width 1.016) (layer B.Cu) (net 1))
 (segment (start 156.718 123.19) (end 153.924 120.396) (width 1.016) (layer B.Cu) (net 1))
 (segment (start 134.112 124.968) (end 134.112 142.494) (width 1.016) (layer B.Cu) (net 1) (status 400000))
 (segment (start 147.53 106.128) (end 147.53 104.12) (width 1.016) (layer B.Cu) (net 1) (status 800000))
 (segment (start 149.606 108.204) (end 147.53 106.128) (width 1.016) (layer B.Cu) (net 1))
 (segment (start 153.162 108.204) (end 149.606 108.204) (width 1.016) (layer B.Cu) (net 1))
 (segment (start 156.972 112.014) (end 153.162 108.204) (width 1.016) (layer B.Cu) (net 1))
 (segment (start 156.972 145.034) (end 156.972 136.906) (width 1.016) (layer B.Cu) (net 1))
 (segment (start 156.972 136.906) (end 156.972 123.19) (width 1.016) (layer B.Cu) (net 1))
 (segment (start 156.972 123.19) (end 156.972 112.014) (width 1.016) (layer B.Cu) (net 1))
 (segment (start 153.416 148.59) (end 156.972 145.034) (width 1.016) (layer B.Cu) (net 1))
 (segment (start 140.208 148.59) (end 144.78 148.59) (width 1.016) (layer B.Cu) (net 1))
 (segment (start 144.78 148.59) (end 153.416 148.59) (width 1.016) (layer B.Cu) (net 1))
 (segment (start 134.112 142.494) (end 140.208 148.59) (width 1.016) (layer B.Cu) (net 1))
 (segment (start 142.03 104.12) (end 147.53 104.12) (width 1.016) (layer B.Cu) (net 1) (status C00000))
 (segment (start 142.03 116.82) (end 147.53 116.82) (width 1.016) (layer B.Cu) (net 1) (status C00000))
 (segment (start 142.03 129.52) (end 147.53 129.52) (width 1.016) (layer B.Cu) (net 1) (status C00000))
 (segment (start 142.03 142.22) (end 147.53 142.22) (width 1.016) (layer B.Cu) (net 1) (status C00000))
 (segment (start 161.817 101) (end 161.817 105.1) (width 1.016) (layer B.Cu) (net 8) (status C00000))
 (segment (start 161.817 105.1) (end 161.942 105.225) (width 1.016) (layer B.Cu) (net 8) (status C00000))
 (segment (start 161.942 105.225) (end 161.942 113.394) (width 1.016) (layer B.Cu) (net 8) (status C00000))
 (segment (start 161.942 113.394) (end 161.798 113.538) (width 1.016) (layer B.Cu) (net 8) (status C00000))
 (segment (start 161.798 113.538) (end 161.798 117.602) (width 1.016) (layer B.Cu) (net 8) (status C00000))
 (segment (start 161.798 117.602) (end 162.052 117.856) (width 1.016) (layer B.Cu) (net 8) (status C00000))
 (segment (start 162.052 117.856) (end 162.052 126.746) (width 1.016) (layer B.Cu) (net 8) (status C00000))
 (segment (start 162.052 126.746) (end 162.052 131.064) (width 1.016) (layer B.Cu) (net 8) (status C00000))
 (segment (start 162.052 131.064) (end 162.052 139.7) (width 1.016) (layer B.Cu) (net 8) (status C00000))
 (segment (start 162.052 139.7) (end 162.306 139.954) (width 1.016) (layer B.Cu) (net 8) (status C00000))
 (segment (start 162.306 144.272) (end 162.306 139.954) (width 1.016) (layer B.Cu) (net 8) (status C00000))
 (segment (start 134.112 122.968) (end 133.064 122.968) (width 1.016) (layer B.Cu) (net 8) (status 400000))
 (segment (start 162.306 147.574) (end 162.306 144.272) (width 1.016) (layer B.Cu) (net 8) (status 800000))
 (segment (start 159.512 150.368) (end 162.306 147.574) (width 1.016) (layer B.Cu) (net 8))
 (segment (start 139.7 150.368) (end 159.512 150.368) (width 1.016) (layer B.Cu) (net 8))
 (segment (start 132.334 143.002) (end 139.7 150.368) (width 1.016) (layer B.Cu) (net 8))
 (segment (start 132.334 123.698) (end 132.334 143.002) (width 1.016) (layer B.Cu) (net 8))
 (segment (start 133.064 122.968) (end 132.334 123.698) (width 1.016) (layer B.Cu) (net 8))
 (segment (start 134.112 120.968) (end 135.7 120.968) (width 1.016) (layer B.Cu) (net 9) (status 400000))
 (segment (start 139.7 137.39) (end 142.03 139.72) (width 1.016) (layer B.Cu) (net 9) (status 800000))
 (segment (start 139.7 124.968) (end 139.7 137.39) (width 1.016) (layer B.Cu) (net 9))
 (segment (start 135.7 120.968) (end 139.7 124.968) (width 1.016) (layer B.Cu) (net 9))
 (segment (start 152.146 139.954) (end 152.146 138.938) (width 1.016) (layer B.Cu) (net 9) (status 400000))
 (segment (start 145.098 136.652) (end 142.03 139.72) (width 1.016) (layer B.Cu) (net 9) (status 800000))
 (segment (start 149.86 136.652) (end 145.098 136.652) (width 1.016) (layer B.Cu) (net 9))
 (segment (start 152.146 138.938) (end 149.86 136.652) (width 1.016) (layer B.Cu) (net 9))
 (segment (start 134.112 118.968) (end 138.018 118.968) (width 1.016) (layer B.Cu) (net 2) (status 400000))
 (segment (start 142.03 122.98) (end 142.03 127.02) (width 1.016) (layer B.Cu) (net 2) (status 800000))
 (segment (start 138.018 118.968) (end 142.03 122.98) (width 1.016) (layer B.Cu) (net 2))
 (segment (start 151.892 126.746) (end 151.892 126.238) (width 1.016) (layer B.Cu) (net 2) (status C00000))
 (segment (start 151.892 126.238) (end 150.114 124.46) (width 1.016) (layer B.Cu) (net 2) (status 400000))
 (segment (start 150.114 124.46) (end 144.59 124.46) (width 1.016) (layer B.Cu) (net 2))
 (segment (start 144.59 124.46) (end 142.03 127.02) (width 1.016) (layer B.Cu) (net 2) (status 800000))
 (segment (start 142.03 114.32) (end 139.426 114.32) (width 1.016) (layer B.Cu) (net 4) (status 400000))
 (segment (start 136.778 116.968) (end 134.112 116.968) (width 1.016) (layer B.Cu) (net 4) (status 800000))
 (segment (start 139.426 114.32) (end 136.778 116.968) (width 1.016) (layer B.Cu) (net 4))
 (segment (start 151.638 113.538) (end 151.638 113.284) (width 1.016) (layer B.Cu) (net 4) (status C00000))
 (segment (start 151.638 113.284) (end 150.368 112.014) (width 1.016) (layer B.Cu) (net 4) (status 400000))
 (segment (start 150.368 112.014) (end 144.336 112.014) (width 1.016) (layer B.Cu) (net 4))
 (segment (start 144.336 112.014) (end 142.03 114.32) (width 1.016) (layer B.Cu) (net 4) (status 800000))
 (segment (start 142.03 101.62) (end 140.95 101.62) (width 1.016) (layer B.Cu) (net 6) (status 400000))
 (segment (start 134.112 108.458) (end 134.112 114.968) (width 1.016) (layer B.Cu) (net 6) (status 800000))
 (segment (start 140.95 101.62) (end 134.112 108.458) (width 1.016) (layer B.Cu) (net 6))
 (segment (start 151.657 101) (end 151.657 100.349) (width 1.016) (layer B.Cu) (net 6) (status C00000))
 (segment (start 151.657 100.349) (end 150.368 99.06) (width 1.016) (layer B.Cu) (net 6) (status 400000))
 (segment (start 150.368 99.06) (end 144.59 99.06) (width 1.016) (layer B.Cu) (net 6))
 (segment (start 144.59 99.06) (end 142.03 101.62) (width 1.016) (layer B.Cu) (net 6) (status 800000))
 (segment (start 151.782 105.225) (end 151.782 104.538) (width 1.016) (layer B.Cu) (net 7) (status C00000))
 (segment (start 151.782 104.538) (end 148.864 101.62) (width 1.016) (layer B.Cu) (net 7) (status 400000))
 (segment (start 148.864 101.62) (end 147.53 101.62) (width 1.016) (layer B.Cu) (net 7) (status 800000))
 (segment (start 147.53 101.62) (end 147.34 101.62) (width 0.25) (layer B.Cu) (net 7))
 (segment (start 151.892 117.856) (end 151.892 116.84) (width 1.016) (layer B.Cu) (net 5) (status 400000))
 (segment (start 149.372 114.32) (end 147.53 114.32) (width 1.016) (layer B.Cu) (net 5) (status 800000))
 (segment (start 151.892 116.84) (end 149.372 114.32) (width 1.016) (layer B.Cu) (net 5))
 (segment (start 151.892 131.064) (end 151.892 130.048) (width 1.016) (layer B.Cu) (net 3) (status 400000))
 (segment (start 148.864 127.02) (end 147.53 127.02) (width 1.016) (layer B.Cu) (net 3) (status 800000))
 (segment (start 151.892 130.048) (end 148.864 127.02) (width 1.016) (layer B.Cu) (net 3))
 (segment (start 152.146 144.272) (end 152.146 143.256) (width 1.016) (layer B.Cu) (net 10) (status 400000))
 (segment (start 148.61 139.72) (end 147.53 139.72) (width 1.016) (layer B.Cu) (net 10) (status 800000))
 (segment (start 152.146 143.256) (end 148.61 139.72) (width 1.016) (layer B.Cu) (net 10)))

